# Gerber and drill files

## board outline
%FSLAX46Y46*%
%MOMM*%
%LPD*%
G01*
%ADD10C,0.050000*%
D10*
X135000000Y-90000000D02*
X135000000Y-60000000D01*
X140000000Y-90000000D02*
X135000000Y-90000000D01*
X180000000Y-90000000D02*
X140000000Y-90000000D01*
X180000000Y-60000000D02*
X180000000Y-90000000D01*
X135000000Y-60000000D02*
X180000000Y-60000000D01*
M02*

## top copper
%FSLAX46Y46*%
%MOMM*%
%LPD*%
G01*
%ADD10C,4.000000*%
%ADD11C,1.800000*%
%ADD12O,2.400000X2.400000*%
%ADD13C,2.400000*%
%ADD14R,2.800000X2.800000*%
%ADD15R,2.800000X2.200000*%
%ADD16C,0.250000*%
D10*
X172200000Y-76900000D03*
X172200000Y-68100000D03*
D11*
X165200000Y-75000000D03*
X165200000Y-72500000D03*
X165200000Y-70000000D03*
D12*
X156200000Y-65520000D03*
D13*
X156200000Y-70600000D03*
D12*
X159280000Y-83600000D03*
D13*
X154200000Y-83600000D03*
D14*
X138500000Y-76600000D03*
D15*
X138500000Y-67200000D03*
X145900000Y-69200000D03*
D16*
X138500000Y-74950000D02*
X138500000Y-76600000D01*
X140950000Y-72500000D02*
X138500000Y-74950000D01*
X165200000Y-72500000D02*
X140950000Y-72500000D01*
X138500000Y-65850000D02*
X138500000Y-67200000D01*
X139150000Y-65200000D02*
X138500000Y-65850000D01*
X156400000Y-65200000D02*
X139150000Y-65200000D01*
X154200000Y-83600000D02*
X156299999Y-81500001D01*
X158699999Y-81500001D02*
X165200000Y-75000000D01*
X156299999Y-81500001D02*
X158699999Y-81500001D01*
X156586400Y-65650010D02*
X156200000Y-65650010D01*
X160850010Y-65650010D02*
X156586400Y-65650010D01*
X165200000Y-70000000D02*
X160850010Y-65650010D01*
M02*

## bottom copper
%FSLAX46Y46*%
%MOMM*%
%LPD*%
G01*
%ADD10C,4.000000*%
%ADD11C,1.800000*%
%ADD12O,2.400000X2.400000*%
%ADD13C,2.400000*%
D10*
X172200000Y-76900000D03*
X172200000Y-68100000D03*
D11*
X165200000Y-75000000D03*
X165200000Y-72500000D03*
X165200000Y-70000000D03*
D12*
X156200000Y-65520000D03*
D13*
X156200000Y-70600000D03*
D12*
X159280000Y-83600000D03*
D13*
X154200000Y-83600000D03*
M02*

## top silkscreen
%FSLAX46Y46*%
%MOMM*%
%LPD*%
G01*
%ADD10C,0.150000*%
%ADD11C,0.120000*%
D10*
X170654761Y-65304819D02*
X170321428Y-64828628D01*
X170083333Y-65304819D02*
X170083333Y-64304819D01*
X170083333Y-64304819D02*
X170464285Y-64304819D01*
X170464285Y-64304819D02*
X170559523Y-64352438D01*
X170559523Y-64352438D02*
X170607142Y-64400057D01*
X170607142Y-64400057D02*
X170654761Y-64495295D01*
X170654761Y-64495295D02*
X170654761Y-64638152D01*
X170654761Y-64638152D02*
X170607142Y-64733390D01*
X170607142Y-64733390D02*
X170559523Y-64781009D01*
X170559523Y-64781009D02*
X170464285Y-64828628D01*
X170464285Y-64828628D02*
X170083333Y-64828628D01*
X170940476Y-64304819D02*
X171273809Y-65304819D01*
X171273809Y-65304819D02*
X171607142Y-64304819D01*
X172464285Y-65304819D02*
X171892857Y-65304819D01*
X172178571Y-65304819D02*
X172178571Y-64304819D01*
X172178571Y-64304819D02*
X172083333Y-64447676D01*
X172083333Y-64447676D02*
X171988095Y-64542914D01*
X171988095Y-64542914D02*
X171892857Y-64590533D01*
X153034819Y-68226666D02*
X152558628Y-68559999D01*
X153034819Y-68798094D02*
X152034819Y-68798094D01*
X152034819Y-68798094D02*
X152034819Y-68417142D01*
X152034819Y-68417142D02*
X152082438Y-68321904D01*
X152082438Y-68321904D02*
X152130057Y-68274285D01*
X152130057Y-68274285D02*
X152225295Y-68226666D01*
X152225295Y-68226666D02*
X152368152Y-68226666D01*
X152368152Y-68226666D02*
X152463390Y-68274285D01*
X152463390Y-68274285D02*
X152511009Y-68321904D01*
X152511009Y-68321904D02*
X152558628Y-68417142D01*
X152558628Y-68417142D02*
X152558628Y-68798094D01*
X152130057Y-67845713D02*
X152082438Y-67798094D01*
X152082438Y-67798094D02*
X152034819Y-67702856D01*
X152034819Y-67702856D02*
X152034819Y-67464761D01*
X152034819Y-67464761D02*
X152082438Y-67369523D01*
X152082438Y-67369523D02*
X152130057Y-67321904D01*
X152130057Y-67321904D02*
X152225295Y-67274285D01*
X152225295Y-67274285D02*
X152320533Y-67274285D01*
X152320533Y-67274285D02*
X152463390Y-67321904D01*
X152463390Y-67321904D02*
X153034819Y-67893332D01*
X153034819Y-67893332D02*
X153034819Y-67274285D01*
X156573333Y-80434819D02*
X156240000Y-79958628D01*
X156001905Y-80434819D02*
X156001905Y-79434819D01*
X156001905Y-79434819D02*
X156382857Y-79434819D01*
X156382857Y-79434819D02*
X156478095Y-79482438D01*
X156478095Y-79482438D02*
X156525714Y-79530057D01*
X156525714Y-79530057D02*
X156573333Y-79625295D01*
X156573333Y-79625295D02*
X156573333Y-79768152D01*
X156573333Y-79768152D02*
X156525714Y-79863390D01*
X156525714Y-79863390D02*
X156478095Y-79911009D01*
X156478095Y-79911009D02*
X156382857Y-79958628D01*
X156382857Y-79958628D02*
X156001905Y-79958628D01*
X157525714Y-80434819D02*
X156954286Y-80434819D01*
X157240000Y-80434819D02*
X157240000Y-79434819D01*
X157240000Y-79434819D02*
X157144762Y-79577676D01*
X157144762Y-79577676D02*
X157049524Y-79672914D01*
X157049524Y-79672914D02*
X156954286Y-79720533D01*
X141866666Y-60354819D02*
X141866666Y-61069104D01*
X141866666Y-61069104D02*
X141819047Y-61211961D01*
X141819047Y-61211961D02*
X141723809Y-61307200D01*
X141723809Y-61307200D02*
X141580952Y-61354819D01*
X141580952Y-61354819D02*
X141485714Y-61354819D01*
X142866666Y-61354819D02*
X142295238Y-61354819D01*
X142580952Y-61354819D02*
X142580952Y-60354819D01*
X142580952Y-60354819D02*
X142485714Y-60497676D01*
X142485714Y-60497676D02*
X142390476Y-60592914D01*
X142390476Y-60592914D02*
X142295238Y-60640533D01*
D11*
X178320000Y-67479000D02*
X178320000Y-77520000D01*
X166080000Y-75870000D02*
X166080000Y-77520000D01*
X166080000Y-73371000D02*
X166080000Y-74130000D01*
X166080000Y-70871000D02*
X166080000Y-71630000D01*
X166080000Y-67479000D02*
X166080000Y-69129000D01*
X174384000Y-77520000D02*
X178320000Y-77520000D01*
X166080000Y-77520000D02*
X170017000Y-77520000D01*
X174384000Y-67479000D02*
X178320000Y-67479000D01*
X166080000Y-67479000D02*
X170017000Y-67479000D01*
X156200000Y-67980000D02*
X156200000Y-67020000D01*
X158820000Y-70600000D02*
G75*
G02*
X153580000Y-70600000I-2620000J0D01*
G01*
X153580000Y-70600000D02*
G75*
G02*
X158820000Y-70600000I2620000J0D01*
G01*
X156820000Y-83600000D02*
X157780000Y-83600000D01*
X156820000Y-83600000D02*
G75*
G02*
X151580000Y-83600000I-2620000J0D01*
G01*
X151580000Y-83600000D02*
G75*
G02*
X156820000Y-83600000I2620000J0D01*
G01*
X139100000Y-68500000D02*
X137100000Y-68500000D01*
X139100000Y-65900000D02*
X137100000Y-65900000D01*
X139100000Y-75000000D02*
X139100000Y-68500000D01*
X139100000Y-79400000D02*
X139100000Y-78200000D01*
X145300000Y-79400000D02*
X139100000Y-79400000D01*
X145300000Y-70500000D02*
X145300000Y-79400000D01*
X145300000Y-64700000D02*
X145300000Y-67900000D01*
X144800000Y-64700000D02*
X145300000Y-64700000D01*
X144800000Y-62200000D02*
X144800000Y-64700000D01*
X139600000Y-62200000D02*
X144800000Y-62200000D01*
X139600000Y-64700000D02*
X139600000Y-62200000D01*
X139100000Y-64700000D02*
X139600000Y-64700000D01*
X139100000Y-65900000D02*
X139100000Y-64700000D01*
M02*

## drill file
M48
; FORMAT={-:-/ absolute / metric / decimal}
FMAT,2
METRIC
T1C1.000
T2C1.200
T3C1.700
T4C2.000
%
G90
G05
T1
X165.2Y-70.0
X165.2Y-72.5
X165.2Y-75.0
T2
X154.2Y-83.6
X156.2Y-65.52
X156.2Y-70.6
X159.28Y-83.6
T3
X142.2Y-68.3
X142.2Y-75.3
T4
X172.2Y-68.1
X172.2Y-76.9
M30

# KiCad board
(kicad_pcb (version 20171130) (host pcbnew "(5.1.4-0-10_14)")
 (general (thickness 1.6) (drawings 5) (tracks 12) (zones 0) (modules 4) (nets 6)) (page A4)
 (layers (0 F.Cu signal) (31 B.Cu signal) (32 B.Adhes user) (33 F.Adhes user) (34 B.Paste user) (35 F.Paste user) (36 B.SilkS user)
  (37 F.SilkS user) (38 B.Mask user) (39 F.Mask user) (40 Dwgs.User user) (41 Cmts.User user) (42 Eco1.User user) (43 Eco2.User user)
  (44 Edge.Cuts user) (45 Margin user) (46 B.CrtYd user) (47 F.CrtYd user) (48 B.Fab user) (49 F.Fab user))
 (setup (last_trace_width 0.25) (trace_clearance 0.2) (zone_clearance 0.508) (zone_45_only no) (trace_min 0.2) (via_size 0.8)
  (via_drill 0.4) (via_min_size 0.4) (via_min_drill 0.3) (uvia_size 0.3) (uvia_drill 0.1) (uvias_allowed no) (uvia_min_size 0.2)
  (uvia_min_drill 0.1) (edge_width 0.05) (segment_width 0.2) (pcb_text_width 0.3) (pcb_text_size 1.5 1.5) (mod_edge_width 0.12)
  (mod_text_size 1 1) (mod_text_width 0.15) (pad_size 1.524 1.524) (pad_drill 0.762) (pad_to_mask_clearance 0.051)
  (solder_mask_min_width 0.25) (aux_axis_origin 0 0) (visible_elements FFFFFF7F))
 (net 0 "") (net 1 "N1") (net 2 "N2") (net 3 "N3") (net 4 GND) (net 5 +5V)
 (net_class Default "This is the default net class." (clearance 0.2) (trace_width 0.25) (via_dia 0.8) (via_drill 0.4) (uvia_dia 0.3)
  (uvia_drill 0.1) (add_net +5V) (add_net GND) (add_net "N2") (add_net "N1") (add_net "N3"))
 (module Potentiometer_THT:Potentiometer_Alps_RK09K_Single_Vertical (layer F.Cu) (at 165.2 75)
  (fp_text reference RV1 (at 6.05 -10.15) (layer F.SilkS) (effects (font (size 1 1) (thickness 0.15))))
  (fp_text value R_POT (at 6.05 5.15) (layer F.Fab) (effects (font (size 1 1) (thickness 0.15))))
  (fp_line (start 13.12 -7.521) (end 13.12 2.52) (layer F.SilkS) (width 0.12))
  (fp_line (start 0.88 0.87) (end 0.88 2.52) (layer F.SilkS) (width 0.12))
  (fp_line (start 0.88 -1.629) (end 0.88 -0.87) (layer F.SilkS) (width 0.12))
  (fp_line (start 0.88 -4.129) (end 0.88 -3.37) (layer F.SilkS) (width 0.12))
  (fp_line (start 0.88 -7.521) (end 0.88 -5.871) (layer F.SilkS) (width 0.12))
  (fp_line (start 9.184 2.52) (end 13.12 2.52) (layer F.SilkS) (width 0.12))
  (fp_line (start 0.88 2.52) (end 4.817 2.52) (layer F.SilkS) (width 0.12))
  (fp_line (start 9.184 -7.521) (end 13.12 -7.521) (layer F.SilkS) (width 0.12))
  (fp_line (start 0.88 -7.521) (end 4.817 -7.521) (layer F.SilkS) (width 0.12))
  (pad "" np_thru_hole circle (at 7 1.9) (size 4 4) (drill 2) (layers *.Cu *.Mask))
  (pad "" np_thru_hole circle (at 7 -6.9) (size 4 4) (drill 2) (layers *.Cu *.Mask))
  (pad 1 thru_hole circle (at 0 0) (size 1.8 1.8) (drill 1) (layers *.Cu *.Mask) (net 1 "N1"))
  (pad 2 thru_hole circle (at 0 -2.5) (size 1.8 1.8) (drill 1) (layers *.Cu *.Mask) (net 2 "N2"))
  (pad 3 thru_hole circle (at 0 -5) (size 1.8 1.8) (drill 1) (layers *.Cu *.Mask) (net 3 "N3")))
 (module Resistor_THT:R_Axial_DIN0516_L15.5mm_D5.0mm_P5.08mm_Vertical (layer F.Cu) (at 156.2 70.6 90)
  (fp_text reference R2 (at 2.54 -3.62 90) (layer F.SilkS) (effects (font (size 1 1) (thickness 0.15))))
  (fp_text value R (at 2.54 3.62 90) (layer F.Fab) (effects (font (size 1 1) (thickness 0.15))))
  (fp_line (start 2.62 0) (end 3.58 0) (layer F.SilkS) (width 0.12))
  (fp_circle (center 0 0) (end 2.62 0) (layer F.SilkS) (width 0.12))
  (pad 2 thru_hole oval (at 5.08 0 90) (size 2.4 2.4) (drill 1.2) (layers *.Cu *.Mask) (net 3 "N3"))
  (pad 1 thru_hole circle (at 0 0 90) (size 2.4 2.4) (drill 1.2) (layers *.Cu *.Mask) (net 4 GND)))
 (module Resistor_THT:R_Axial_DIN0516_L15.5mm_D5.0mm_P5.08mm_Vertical (layer F.Cu) (at 154.2 83.6)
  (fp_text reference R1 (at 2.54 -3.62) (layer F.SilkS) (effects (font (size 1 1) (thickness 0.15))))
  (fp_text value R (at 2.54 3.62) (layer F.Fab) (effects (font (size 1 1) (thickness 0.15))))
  (fp_line (start 2.62 0) (end 3.58 0) (layer F.SilkS) (width 0.12))
  (fp_circle (center 0 0) (end 2.62 0) (layer F.SilkS) (width 0.12))
  (pad 2 thru_hole oval (at 5.08 0) (size 2.4 2.4) (drill 1.2) (layers *.Cu *.Mask) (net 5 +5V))
  (pad 1 thru_hole circle (at 0 0) (size 2.4 2.4) (drill 1.2) (layers *.Cu *.Mask) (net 1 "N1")))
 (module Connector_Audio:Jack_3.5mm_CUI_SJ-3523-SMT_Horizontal (layer F.Cu) (at 142.2 70.8)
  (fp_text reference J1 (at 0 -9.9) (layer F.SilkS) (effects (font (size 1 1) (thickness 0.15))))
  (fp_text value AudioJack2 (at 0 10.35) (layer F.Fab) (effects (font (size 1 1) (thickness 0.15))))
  (fp_line (start -3.1 -2.3) (end -5.1 -2.3) (layer F.SilkS) (width 0.12))
  (fp_line (start -3.1 -4.9) (end -5.1 -4.9) (layer F.SilkS) (width 0.12))
  (fp_line (start -3.1 4.2) (end -3.1 -2.3) (layer F.SilkS) (width 0.12))
  (fp_line (start -3.1 8.6) (end -3.1 7.4) (layer F.SilkS) (width 0.12))
  (fp_line (start 3.1 8.6) (end -3.1 8.6) (layer F.SilkS) (width 0.12))
  (fp_line (start 3.1 -0.3) (end 3.1 8.6) (layer F.SilkS) (width 0.12))
  (fp_line (start 3.1 -6.1) (end 3.1 -2.9) (layer F.SilkS) (width 0.12))
  (fp_line (start 2.6 -6.1) (end 3.1 -6.1) (layer F.SilkS) (width 0.12))
  (fp_line (start 2.6 -8.6) (end 2.6 -6.1) (layer F.SilkS) (width 0.12))
  (fp_line (start -2.6 -8.6) (end 2.6 -8.6) (layer F.SilkS) (width 0.12))
  (fp_line (start -2.6 -6.1) (end -2.6 -8.6) (layer F.SilkS) (width 0.12))
  (fp_line (start -3.1 -6.1) (end -2.6 -6.1) (layer F.SilkS) (width 0.12))
  (fp_line (start -3.1 -4.9) (end -3.1 -6.1) (layer F.SilkS) (width 0.12))
  (pad "" np_thru_hole circle (at 0 4.5) (size 1.7 1.7) (drill 1.7) (layers *.Cu *.Mask))
  (pad "" np_thru_hole circle (at 0 -2.5) (size 1.7 1.7) (drill 1.7) (layers *.Cu *.Mask))
  (pad T smd rect (at -3.7 5.8) (size 2.8 2.8) (layers F.Cu F.Paste F.Mask) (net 2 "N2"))
  (pad S smd rect (at -3.7 -3.6) (size 2.8 2.2) (layers F.Cu F.Paste F.Mask) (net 4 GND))
  (pad R smd rect (at 3.7 -1.6) (size 2.8 2.2) (layers F.Cu F.Paste F.Mask)))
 (gr_line (start 135 90) (end 135 60) (layer Edge.Cuts) (width 0.05))
 (gr_line (start 140 90) (end 135 90) (layer Edge.Cuts) (width 0.05))
 (gr_line (start 180 90) (end 140 90) (layer Edge.Cuts) (width 0.05))
 (gr_line (start 180 60) (end 180 90) (layer Edge.Cuts) (width 0.05))
 (gr_line (start 135 60) (end 180 60) (layer Edge.Cuts) (width 0.05))
 (segment (start 138.5 74.95) (end 138.5 76.6) (width 0.25) (layer F.Cu) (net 2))
 (segment (start 140.95 72.5) (end 138.5 74.95) (width 0.25) (layer F.Cu) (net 2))
 (segment (start 165.2 72.5) (end 140.95 72.5) (width 0.25) (layer F.Cu) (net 2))
 (segment (start 138.5 65.85) (end 138.5 67.2) (width 0.25) (layer F.Cu) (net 4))
 (segment (start 139.15 65.2) (end 138.5 65.85) (width 0.25) (layer F.Cu) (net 4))
 (segment (start 156.4 65.2) (end 139.15 65.2) (width 0.25) (layer F.Cu) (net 4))
 (segment (start 154.2 83.6) (end 156.299999 81.500001) (width 0.25) (layer F.Cu) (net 1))
 (segment (start 158.699999 81.500001) (end 165.2 75) (width 0.25) (layer F.Cu) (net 1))
 (segment (start 156.299999 81.500001) (end 158.699999 81.500001) (width 0.25) (layer F.Cu) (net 1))
 (segment (start 156.5864 65.65001) (end 156.2 65.65001) (width 0.25) (layer F.Cu) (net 3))
 (segment (start 160.85001 65.65001) (end 156.5864 65.65001) (width 0.25) (layer F.Cu) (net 3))
 (segment (start 165.2 70) (end 160.85001 65.65001) (width 0.25) (layer F.Cu) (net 3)))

